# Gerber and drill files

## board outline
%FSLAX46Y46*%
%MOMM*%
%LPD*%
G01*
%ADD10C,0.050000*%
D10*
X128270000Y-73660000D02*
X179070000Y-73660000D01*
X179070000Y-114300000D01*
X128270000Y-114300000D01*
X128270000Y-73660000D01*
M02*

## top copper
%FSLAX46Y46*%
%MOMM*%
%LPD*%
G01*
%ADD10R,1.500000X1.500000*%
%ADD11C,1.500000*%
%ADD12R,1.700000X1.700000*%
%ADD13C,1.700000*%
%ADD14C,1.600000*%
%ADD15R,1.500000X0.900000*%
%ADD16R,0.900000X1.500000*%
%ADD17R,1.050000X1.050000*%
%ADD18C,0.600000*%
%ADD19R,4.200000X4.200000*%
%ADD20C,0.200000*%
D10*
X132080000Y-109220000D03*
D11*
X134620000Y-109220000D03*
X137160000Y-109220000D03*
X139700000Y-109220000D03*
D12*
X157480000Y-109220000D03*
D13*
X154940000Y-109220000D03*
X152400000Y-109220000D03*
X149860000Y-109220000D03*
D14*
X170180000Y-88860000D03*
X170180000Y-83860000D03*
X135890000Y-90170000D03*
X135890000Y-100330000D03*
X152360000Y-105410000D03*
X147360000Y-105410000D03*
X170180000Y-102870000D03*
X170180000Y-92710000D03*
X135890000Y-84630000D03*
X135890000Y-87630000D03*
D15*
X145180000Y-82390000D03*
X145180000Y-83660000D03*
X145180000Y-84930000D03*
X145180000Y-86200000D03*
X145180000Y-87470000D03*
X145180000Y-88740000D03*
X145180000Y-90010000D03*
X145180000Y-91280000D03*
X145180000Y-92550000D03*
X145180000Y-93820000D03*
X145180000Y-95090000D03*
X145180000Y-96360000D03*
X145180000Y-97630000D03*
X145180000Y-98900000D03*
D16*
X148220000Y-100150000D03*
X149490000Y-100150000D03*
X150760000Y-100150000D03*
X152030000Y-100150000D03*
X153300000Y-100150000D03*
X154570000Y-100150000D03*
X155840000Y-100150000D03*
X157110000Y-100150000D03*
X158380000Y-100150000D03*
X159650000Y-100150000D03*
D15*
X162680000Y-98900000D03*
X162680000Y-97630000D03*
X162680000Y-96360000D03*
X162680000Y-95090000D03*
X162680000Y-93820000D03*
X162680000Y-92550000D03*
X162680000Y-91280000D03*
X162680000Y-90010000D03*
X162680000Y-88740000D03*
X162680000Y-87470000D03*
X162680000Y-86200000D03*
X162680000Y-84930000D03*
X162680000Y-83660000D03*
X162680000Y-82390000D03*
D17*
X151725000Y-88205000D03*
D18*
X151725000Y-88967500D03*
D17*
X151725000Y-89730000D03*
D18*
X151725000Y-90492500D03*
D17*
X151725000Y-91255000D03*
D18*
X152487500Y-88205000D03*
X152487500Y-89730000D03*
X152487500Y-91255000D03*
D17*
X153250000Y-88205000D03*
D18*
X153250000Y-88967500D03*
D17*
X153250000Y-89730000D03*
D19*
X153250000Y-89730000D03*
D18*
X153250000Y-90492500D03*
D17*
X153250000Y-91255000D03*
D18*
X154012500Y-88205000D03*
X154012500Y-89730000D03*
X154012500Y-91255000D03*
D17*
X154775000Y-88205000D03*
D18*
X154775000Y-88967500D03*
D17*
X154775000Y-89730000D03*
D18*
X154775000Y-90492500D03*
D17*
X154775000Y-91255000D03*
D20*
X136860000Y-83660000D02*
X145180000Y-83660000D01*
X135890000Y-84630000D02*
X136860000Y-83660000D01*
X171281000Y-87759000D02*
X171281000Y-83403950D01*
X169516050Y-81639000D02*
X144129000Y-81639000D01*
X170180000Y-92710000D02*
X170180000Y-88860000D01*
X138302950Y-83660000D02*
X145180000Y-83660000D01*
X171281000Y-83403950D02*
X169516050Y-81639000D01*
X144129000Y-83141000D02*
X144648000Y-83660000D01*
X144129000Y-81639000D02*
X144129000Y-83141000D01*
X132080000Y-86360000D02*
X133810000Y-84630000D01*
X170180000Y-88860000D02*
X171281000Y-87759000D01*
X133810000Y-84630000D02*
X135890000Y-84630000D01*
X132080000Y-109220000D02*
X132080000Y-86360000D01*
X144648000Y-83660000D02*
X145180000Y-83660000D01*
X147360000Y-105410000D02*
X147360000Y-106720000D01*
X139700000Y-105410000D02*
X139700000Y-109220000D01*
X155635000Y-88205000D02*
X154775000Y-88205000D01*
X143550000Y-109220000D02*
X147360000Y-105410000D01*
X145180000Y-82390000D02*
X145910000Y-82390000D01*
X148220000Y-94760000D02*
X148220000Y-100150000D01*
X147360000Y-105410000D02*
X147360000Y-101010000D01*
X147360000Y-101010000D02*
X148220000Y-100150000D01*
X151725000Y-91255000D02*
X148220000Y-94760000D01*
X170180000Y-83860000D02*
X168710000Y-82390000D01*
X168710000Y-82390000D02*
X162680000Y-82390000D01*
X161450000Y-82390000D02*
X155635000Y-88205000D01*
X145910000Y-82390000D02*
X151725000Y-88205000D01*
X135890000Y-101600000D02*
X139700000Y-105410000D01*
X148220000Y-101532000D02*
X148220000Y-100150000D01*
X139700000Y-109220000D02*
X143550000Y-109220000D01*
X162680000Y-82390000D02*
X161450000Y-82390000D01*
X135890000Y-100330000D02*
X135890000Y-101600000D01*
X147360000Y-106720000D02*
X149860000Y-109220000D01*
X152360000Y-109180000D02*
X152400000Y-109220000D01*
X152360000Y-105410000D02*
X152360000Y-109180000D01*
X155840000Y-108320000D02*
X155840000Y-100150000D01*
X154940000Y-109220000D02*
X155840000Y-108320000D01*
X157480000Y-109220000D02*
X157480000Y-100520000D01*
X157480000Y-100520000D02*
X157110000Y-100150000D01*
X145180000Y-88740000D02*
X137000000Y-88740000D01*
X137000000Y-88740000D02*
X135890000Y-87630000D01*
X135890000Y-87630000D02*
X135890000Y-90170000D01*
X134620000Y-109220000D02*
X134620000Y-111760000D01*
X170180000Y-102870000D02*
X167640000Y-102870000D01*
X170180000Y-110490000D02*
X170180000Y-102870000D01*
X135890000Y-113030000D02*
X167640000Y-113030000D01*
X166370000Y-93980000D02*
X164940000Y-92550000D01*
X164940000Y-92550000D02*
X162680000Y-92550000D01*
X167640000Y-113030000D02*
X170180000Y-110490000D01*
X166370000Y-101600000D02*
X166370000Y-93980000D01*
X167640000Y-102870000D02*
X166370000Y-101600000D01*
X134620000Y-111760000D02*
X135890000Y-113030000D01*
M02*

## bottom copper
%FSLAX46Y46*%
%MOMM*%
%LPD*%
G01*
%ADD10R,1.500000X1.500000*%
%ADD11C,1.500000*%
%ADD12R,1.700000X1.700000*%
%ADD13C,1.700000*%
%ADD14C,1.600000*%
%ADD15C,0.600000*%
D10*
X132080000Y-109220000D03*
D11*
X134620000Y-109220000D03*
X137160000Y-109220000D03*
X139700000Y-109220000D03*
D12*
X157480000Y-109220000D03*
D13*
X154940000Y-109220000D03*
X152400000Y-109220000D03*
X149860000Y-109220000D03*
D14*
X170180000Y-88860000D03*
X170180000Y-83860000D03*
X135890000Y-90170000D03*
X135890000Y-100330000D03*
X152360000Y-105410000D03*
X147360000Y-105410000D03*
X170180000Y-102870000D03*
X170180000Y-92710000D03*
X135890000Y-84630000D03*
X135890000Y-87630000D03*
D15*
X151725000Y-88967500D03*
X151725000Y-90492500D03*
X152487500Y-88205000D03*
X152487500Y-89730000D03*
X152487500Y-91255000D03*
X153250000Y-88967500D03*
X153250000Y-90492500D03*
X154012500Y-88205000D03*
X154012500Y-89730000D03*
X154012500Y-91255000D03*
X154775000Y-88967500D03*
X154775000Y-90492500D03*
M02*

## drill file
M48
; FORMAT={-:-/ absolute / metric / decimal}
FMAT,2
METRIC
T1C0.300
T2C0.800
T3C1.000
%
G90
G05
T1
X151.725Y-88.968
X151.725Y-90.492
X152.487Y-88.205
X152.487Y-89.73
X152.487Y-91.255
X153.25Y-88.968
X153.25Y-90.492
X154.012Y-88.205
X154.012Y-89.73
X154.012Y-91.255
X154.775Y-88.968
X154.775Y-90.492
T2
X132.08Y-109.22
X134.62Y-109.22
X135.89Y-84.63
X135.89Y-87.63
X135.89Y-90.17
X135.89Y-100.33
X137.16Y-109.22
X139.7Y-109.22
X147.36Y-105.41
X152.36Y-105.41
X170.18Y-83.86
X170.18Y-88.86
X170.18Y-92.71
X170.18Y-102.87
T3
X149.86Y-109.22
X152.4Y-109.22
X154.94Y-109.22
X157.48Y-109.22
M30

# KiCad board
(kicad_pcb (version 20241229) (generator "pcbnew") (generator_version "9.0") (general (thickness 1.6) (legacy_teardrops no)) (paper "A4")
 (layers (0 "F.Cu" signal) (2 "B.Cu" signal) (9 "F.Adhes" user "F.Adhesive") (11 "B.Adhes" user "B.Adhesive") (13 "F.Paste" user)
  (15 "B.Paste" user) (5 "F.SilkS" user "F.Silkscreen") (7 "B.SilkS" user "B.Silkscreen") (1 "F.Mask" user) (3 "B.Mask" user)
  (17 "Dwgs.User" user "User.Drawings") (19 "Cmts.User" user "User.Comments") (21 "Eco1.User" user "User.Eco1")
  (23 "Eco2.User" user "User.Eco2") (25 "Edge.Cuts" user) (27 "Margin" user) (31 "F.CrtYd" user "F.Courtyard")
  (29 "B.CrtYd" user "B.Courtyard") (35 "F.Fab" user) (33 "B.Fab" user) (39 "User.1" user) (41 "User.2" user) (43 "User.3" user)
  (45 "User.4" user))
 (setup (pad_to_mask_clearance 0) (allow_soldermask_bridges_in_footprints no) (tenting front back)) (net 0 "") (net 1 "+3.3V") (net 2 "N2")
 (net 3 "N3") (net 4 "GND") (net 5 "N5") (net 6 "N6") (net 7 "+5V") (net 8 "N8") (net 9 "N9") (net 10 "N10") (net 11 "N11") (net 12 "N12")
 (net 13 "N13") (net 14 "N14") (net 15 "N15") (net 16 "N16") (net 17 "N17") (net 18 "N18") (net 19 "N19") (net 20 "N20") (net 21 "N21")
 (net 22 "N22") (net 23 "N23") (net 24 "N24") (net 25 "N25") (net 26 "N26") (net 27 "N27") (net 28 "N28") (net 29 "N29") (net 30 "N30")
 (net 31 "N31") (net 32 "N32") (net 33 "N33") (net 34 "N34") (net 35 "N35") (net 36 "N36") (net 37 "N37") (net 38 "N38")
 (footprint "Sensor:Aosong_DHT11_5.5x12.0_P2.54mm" (layer "F.Cu") (at 132.08 109.22 90)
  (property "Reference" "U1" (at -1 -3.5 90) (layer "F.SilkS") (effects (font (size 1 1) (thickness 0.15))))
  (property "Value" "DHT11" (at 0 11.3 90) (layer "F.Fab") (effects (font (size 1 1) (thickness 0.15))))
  (pad "1" thru_hole rect (at 0 0 90) (size 1.5 1.5) (drill 0.8) (layers "*.Cu" "*.Mask") (remove_unused_layers no) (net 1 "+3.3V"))
  (pad "2" thru_hole circle (at 0 2.54 90) (size 1.5 1.5) (drill 0.8) (layers "*.Cu" "*.Mask") (remove_unused_layers no) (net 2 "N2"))
  (pad "3" thru_hole circle (at 0 5.08 90) (size 1.5 1.5) (drill 0.8) (layers "*.Cu" "*.Mask") (remove_unused_layers no) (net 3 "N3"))
  (pad "4" thru_hole circle (at 0 7.62 90) (size 1.5 1.5) (drill 0.8) (layers "*.Cu" "*.Mask") (remove_unused_layers no) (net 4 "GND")))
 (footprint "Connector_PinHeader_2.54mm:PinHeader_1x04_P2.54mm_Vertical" (layer "F.Cu") (at 157.48 109.22 -90)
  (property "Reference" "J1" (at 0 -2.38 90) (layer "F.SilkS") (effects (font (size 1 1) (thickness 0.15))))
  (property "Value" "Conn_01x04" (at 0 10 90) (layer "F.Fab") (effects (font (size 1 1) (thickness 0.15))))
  (pad "1" thru_hole rect (at 0 0 270) (size 1.7 1.7) (drill 1) (layers "*.Cu" "*.Mask") (remove_unused_layers no) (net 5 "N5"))
  (pad "2" thru_hole circle (at 0 2.54 270) (size 1.7 1.7) (drill 1) (layers "*.Cu" "*.Mask") (remove_unused_layers no) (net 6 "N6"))
  (pad "3" thru_hole circle (at 0 5.08 270) (size 1.7 1.7) (drill 1) (layers "*.Cu" "*.Mask") (remove_unused_layers no) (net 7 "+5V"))
  (pad "4" thru_hole circle (at 0 7.62 270) (size 1.7 1.7) (drill 1) (layers "*.Cu" "*.Mask") (remove_unused_layers no) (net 4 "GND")))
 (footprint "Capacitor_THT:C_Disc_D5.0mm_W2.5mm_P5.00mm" (layer "F.Cu") (at 170.18 88.86 90)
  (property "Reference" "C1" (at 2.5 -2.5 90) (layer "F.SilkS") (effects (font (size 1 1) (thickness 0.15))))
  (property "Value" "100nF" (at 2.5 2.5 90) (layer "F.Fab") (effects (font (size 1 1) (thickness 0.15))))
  (pad "1" thru_hole circle (at 0 0 90) (size 1.6 1.6) (drill 0.8) (layers "*.Cu" "*.Mask") (remove_unused_layers no) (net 1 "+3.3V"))
  (pad "2" thru_hole circle (at 5 0 90) (size 1.6 1.6) (drill 0.8) (layers "*.Cu" "*.Mask") (remove_unused_layers no) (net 4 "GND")))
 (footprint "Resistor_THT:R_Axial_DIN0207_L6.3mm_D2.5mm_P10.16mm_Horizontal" (layer "F.Cu") (at 135.89 90.17 -90)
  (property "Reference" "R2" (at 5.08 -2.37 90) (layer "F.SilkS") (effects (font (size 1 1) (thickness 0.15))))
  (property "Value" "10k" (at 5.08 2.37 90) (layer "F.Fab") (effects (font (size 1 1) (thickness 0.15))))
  (pad "1" thru_hole circle (at 0 0 270) (size 1.6 1.6) (drill 0.8) (layers "*.Cu" "*.Mask") (remove_unused_layers no) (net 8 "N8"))
  (pad "2" thru_hole circle (at 10.16 0 270) (size 1.6 1.6) (drill 0.8) (layers "*.Cu" "*.Mask") (remove_unused_layers no) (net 4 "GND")))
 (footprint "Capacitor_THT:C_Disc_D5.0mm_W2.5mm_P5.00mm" (layer "F.Cu") (at 152.36 105.41 180)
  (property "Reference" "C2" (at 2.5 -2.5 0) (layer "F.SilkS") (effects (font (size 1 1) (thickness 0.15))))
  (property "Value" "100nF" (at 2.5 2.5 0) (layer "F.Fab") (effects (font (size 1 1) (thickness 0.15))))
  (pad "1" thru_hole circle (at 0 0 180) (size 1.6 1.6) (drill 0.8) (layers "*.Cu" "*.Mask") (remove_unused_layers no) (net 7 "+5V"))
  (pad "2" thru_hole circle (at 5 0 180) (size 1.6 1.6) (drill 0.8) (layers "*.Cu" "*.Mask") (remove_unused_layers no) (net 4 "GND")))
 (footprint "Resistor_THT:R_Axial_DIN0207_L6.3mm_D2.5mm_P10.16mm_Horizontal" (layer "F.Cu") (at 170.18 102.87 90)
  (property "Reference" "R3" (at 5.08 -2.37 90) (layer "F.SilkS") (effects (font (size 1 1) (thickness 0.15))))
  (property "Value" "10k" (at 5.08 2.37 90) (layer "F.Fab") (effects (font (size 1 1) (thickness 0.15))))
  (pad "1" thru_hole circle (at 0 0 90) (size 1.6 1.6) (drill 0.8) (layers "*.Cu" "*.Mask") (remove_unused_layers no) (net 2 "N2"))
  (pad "2" thru_hole circle (at 10.16 0 90) (size 1.6 1.6) (drill 0.8) (layers "*.Cu" "*.Mask") (remove_unused_layers no) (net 1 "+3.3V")))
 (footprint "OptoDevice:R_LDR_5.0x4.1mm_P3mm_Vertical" (layer "F.Cu") (at 135.89 84.63 -90)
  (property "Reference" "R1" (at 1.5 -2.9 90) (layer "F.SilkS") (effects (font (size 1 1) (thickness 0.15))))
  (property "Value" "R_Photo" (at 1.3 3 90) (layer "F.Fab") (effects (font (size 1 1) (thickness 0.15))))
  (pad "1" thru_hole circle (at 0 0 270) (size 1.6 1.6) (drill 0.8) (layers "*.Cu" "*.Mask") (remove_unused_layers no) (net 1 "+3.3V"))
  (pad "2" thru_hole circle (at 3 0 270) (size 1.6 1.6) (drill 0.8) (layers "*.Cu" "*.Mask") (remove_unused_layers no) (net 8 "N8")))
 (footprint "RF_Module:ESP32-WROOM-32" (layer "F.Cu") (at 153.93 90.64)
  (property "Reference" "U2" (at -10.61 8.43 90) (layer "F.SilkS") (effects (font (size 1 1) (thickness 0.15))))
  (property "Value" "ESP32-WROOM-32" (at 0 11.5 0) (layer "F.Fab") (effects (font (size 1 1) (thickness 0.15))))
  (pad "1" smd rect (at -8.75 -8.25) (size 1.5 0.9) (layers "F.Cu" "F.Mask" "F.Paste") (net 4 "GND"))
  (pad "2" smd rect (at -8.75 -6.98) (size 1.5 0.9) (layers "F.Cu" "F.Mask" "F.Paste") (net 1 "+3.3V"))
  (pad "3" smd rect (at -8.75 -5.71) (size 1.5 0.9) (layers "F.Cu" "F.Mask" "F.Paste") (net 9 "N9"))
  (pad "4" smd rect (at -8.75 -4.44) (size 1.5 0.9) (layers "F.Cu" "F.Mask" "F.Paste") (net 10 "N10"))
  (pad "5" smd rect (at -8.75 -3.17) (size 1.5 0.9) (layers "F.Cu" "F.Mask" "F.Paste") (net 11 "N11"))
  (pad "6" smd rect (at -8.75 -1.9) (size 1.5 0.9) (layers "F.Cu" "F.Mask" "F.Paste") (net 8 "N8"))
  (pad "7" smd rect (at -8.75 -0.63) (size 1.5 0.9) (layers "F.Cu" "F.Mask" "F.Paste") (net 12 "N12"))
  (pad "8" smd rect (at -8.75 0.64) (size 1.5 0.9) (layers "F.Cu" "F.Mask" "F.Paste") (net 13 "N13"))
  (pad "9" smd rect (at -8.75 1.91) (size 1.5 0.9) (layers "F.Cu" "F.Mask" "F.Paste") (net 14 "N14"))
  (pad "10" smd rect (at -8.75 3.18) (size 1.5 0.9) (layers "F.Cu" "F.Mask" "F.Paste") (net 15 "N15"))
  (pad "11" smd rect (at -8.75 4.45) (size 1.5 0.9) (layers "F.Cu" "F.Mask" "F.Paste") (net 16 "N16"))
  (pad "12" smd rect (at -8.75 5.72) (size 1.5 0.9) (layers "F.Cu" "F.Mask" "F.Paste") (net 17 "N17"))
  (pad "13" smd rect (at -8.75 6.99) (size 1.5 0.9) (layers "F.Cu" "F.Mask" "F.Paste") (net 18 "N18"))
  (pad "14" smd rect (at -8.75 8.26) (size 1.5 0.9) (layers "F.Cu" "F.Mask" "F.Paste") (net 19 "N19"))
  (pad "15" smd rect (at -5.71 9.51 90) (size 1.5 0.9) (layers "F.Cu" "F.Mask" "F.Paste") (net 4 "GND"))
  (pad "16" smd rect (at -4.44 9.51 90) (size 1.5 0.9) (layers "F.Cu" "F.Mask" "F.Paste") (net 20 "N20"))
  (pad "17" smd rect (at -3.17 9.51 90) (size 1.5 0.9) (layers "F.Cu" "F.Mask" "F.Paste") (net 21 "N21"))
  (pad "18" smd rect (at -1.9 9.51 90) (size 1.5 0.9) (layers "F.Cu" "F.Mask" "F.Paste") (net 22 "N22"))
  (pad "19" smd rect (at -0.63 9.51 90) (size 1.5 0.9) (layers "F.Cu" "F.Mask" "F.Paste") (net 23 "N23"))
  (pad "20" smd rect (at 0.64 9.51 90) (size 1.5 0.9) (layers "F.Cu" "F.Mask" "F.Paste") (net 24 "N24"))
  (pad "21" smd rect (at 1.91 9.51 90) (size 1.5 0.9) (layers "F.Cu" "F.Mask" "F.Paste") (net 6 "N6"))
  (pad "22" smd rect (at 3.18 9.51 90) (size 1.5 0.9) (layers "F.Cu" "F.Mask" "F.Paste") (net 5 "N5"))
  (pad "23" smd rect (at 4.45 9.51 90) (size 1.5 0.9) (layers "F.Cu" "F.Mask" "F.Paste") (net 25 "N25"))
  (pad "24" smd rect (at 5.72 9.51 90) (size 1.5 0.9) (layers "F.Cu" "F.Mask" "F.Paste") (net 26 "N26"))
  (pad "25" smd rect (at 8.75 8.26) (size 1.5 0.9) (layers "F.Cu" "F.Mask" "F.Paste") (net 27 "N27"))
  (pad "26" smd rect (at 8.75 6.99) (size 1.5 0.9) (layers "F.Cu" "F.Mask" "F.Paste") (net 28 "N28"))
  (pad "27" smd rect (at 8.75 5.72) (size 1.5 0.9) (layers "F.Cu" "F.Mask" "F.Paste") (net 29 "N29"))
  (pad "28" smd rect (at 8.75 4.45) (size 1.5 0.9) (layers "F.Cu" "F.Mask" "F.Paste") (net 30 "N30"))
  (pad "29" smd rect (at 8.75 3.18) (size 1.5 0.9) (layers "F.Cu" "F.Mask" "F.Paste") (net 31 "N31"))
  (pad "30" smd rect (at 8.75 1.91) (size 1.5 0.9) (layers "F.Cu" "F.Mask" "F.Paste") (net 2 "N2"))
  (pad "31" smd rect (at 8.75 0.64) (size 1.5 0.9) (layers "F.Cu" "F.Mask" "F.Paste") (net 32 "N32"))
  (pad "32" smd rect (at 8.75 -0.63) (size 1.5 0.9) (layers "F.Cu" "F.Mask" "F.Paste") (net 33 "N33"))
  (pad "33" smd rect (at 8.75 -1.9) (size 1.5 0.9) (layers "F.Cu" "F.Mask" "F.Paste") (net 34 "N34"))
  (pad "34" smd rect (at 8.75 -3.17) (size 1.5 0.9) (layers "F.Cu" "F.Mask" "F.Paste") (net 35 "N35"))
  (pad "35" smd rect (at 8.75 -4.44) (size 1.5 0.9) (layers "F.Cu" "F.Mask" "F.Paste") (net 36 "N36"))
  (pad "36" smd rect (at 8.75 -5.71) (size 1.5 0.9) (layers "F.Cu" "F.Mask" "F.Paste") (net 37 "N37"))
  (pad "37" smd rect (at 8.75 -6.98) (size 1.5 0.9) (layers "F.Cu" "F.Mask" "F.Paste") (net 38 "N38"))
  (pad "38" smd rect (at 8.75 -8.25) (size 1.5 0.9) (layers "F.Cu" "F.Mask" "F.Paste") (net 4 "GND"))
  (pad "39" smd rect (at -2.205 -2.435) (size 1.05 1.05) (layers "F.Cu" "F.Paste") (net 4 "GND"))
  (pad "39" thru_hole circle (at -2.205 -1.6725) (size 0.6 0.6) (drill 0.3) (layers "*.Cu" "F.Mask") (remove_unused_layers no) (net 4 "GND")
   (zone_connect 2))
  (pad "39" smd rect (at -2.205 -0.91) (size 1.05 1.05) (layers "F.Cu" "F.Paste") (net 4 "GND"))
  (pad "39" thru_hole circle (at -2.205 -0.1475) (size 0.6 0.6) (drill 0.3) (layers "*.Cu" "F.Mask") (remove_unused_layers no) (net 4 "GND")
   (zone_connect 2))
  (pad "39" smd rect (at -2.205 0.615) (size 1.05 1.05) (layers "F.Cu" "F.Paste") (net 4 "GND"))
  (pad "39" thru_hole circle (at -1.4425 -2.435) (size 0.6 0.6) (drill 0.3) (layers "*.Cu" "F.Mask") (remove_unused_layers no) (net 4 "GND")
   (zone_connect 2))
  (pad "39" thru_hole circle (at -1.4425 -0.91) (size 0.6 0.6) (drill 0.3) (layers "*.Cu" "F.Mask") (remove_unused_layers no) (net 4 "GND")
   (zone_connect 2))
  (pad "39" thru_hole circle (at -1.4425 0.615) (size 0.6 0.6) (drill 0.3) (layers "*.Cu" "F.Mask") (remove_unused_layers no) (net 4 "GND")
   (zone_connect 2))
  (pad "39" smd rect (at -0.68 -2.435) (size 1.05 1.05) (layers "F.Cu" "F.Paste") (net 4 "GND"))
  (pad "39" thru_hole circle (at -0.68 -1.6725) (size 0.6 0.6) (drill 0.3) (layers "*.Cu" "F.Mask") (remove_unused_layers no) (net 4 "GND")
   (zone_connect 2))
  (pad "39" smd rect (at -0.68 -0.91) (size 1.05 1.05) (layers "F.Cu" "F.Paste") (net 4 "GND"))
  (pad "39" smd rect (at -0.68 -0.91) (size 4.2 4.2) (layers "F.Cu" "F.Mask") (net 4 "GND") (zone_connect 2))
  (pad "39" thru_hole circle (at -0.68 -0.1475) (size 0.6 0.6) (drill 0.3) (layers "*.Cu" "F.Mask") (remove_unused_layers no) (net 4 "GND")
   (zone_connect 2))
  (pad "39" smd rect (at -0.68 0.615) (size 1.05 1.05) (layers "F.Cu" "F.Paste") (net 4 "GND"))
  (pad "39" thru_hole circle (at 0.0825 -2.435) (size 0.6 0.6) (drill 0.3) (layers "*.Cu" "F.Mask") (remove_unused_layers no) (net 4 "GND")
   (zone_connect 2))
  (pad "39" thru_hole circle (at 0.0825 -0.91) (size 0.6 0.6) (drill 0.3) (layers "*.Cu" "F.Mask") (remove_unused_layers no) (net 4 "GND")
   (zone_connect 2))
  (pad "39" thru_hole circle (at 0.0825 0.615) (size 0.6 0.6) (drill 0.3) (layers "*.Cu" "F.Mask") (remove_unused_layers no) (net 4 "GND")
   (zone_connect 2))
  (pad "39" smd rect (at 0.845 -2.435) (size 1.05 1.05) (layers "F.Cu" "F.Paste") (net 4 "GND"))
  (pad "39" thru_hole circle (at 0.845 -1.6725) (size 0.6 0.6) (drill 0.3) (layers "*.Cu" "F.Mask") (remove_unused_layers no) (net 4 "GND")
   (zone_connect 2))
  (pad "39" smd rect (at 0.845 -0.91) (size 1.05 1.05) (layers "F.Cu" "F.Paste") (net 4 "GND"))
  (pad "39" thru_hole circle (at 0.845 -0.1475) (size 0.6 0.6) (drill 0.3) (layers "*.Cu" "F.Mask") (remove_unused_layers no) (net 4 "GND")
   (zone_connect 2))
  (pad "39" smd rect (at 0.845 0.615) (size 1.05 1.05) (layers "F.Cu" "F.Paste") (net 4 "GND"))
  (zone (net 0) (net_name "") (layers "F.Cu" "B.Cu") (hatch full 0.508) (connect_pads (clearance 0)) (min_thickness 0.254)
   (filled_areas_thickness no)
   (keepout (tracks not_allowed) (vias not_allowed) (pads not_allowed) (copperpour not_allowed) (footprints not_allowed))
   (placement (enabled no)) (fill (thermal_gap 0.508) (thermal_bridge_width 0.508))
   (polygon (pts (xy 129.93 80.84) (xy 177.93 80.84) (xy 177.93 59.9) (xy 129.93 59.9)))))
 (gr_rect (start 128.27 73.66) (end 179.07 114.3) (stroke (width 0.05) (type default)) (fill no) (layer "Edge.Cuts"))
 (segment (start 136.86 83.66) (end 145.18 83.66) (width 0.2) (layer "F.Cu") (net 1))
 (segment (start 135.89 84.63) (end 136.86 83.66) (width 0.2) (layer "F.Cu") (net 1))
 (segment (start 171.281 87.759) (end 171.281 83.40395) (width 0.2) (layer "F.Cu") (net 1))
 (segment (start 169.51605 81.639) (end 144.129 81.639) (width 0.2) (layer "F.Cu") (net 1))
 (segment (start 170.18 92.71) (end 170.18 88.86) (width 0.2) (layer "F.Cu") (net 1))
 (segment (start 138.30295 83.66) (end 145.18 83.66) (width 0.2) (layer "F.Cu") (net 1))
 (segment (start 171.281 83.40395) (end 169.51605 81.639) (width 0.2) (layer "F.Cu") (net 1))
 (segment (start 144.129 83.141) (end 144.648 83.66) (width 0.2) (layer "F.Cu") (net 1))
 (segment (start 144.129 81.639) (end 144.129 83.141) (width 0.2) (layer "F.Cu") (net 1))
 (segment (start 132.08 86.36) (end 133.81 84.63) (width 0.2) (layer "F.Cu") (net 1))
 (segment (start 170.18 88.86) (end 171.281 87.759) (width 0.2) (layer "F.Cu") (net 1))
 (segment (start 133.81 84.63) (end 135.89 84.63) (width 0.2) (layer "F.Cu") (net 1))
 (segment (start 132.08 109.22) (end 132.08 86.36) (width 0.2) (layer "F.Cu") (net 1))
 (segment (start 144.648 83.66) (end 145.18 83.66) (width 0.2) (layer "F.Cu") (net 1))
 (segment (start 147.36 105.41) (end 147.36 106.72) (width 0.2) (layer "F.Cu") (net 4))
 (segment (start 139.7 105.41) (end 139.7 109.22) (width 0.2) (layer "F.Cu") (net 4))
 (segment (start 155.635 88.205) (end 154.775 88.205) (width 0.2) (layer "F.Cu") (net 4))
 (segment (start 143.55 109.22) (end 147.36 105.41) (width 0.2) (layer "F.Cu") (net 4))
 (segment (start 145.18 82.39) (end 145.91 82.39) (width 0.2) (layer "F.Cu") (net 4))
 (segment (start 148.22 94.76) (end 148.22 100.15) (width 0.2) (layer "F.Cu") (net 4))
 (segment (start 147.36 105.41) (end 147.36 101.01) (width 0.2) (layer "F.Cu") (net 4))
 (segment (start 147.36 101.01) (end 148.22 100.15) (width 0.2) (layer "F.Cu") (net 4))
 (segment (start 151.725 91.255) (end 148.22 94.76) (width 0.2) (layer "F.Cu") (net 4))
 (segment (start 170.18 83.86) (end 168.71 82.39) (width 0.2) (layer "F.Cu") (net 4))
 (segment (start 168.71 82.39) (end 162.68 82.39) (width 0.2) (layer "F.Cu") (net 4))
 (segment (start 161.45 82.39) (end 155.635 88.205) (width 0.2) (layer "F.Cu") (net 4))
 (segment (start 145.91 82.39) (end 151.725 88.205) (width 0.2) (layer "F.Cu") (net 4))
 (segment (start 135.89 101.6) (end 139.7 105.41) (width 0.2) (layer "F.Cu") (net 4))
 (segment (start 148.22 101.532) (end 148.22 100.15) (width 0.2) (layer "F.Cu") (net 4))
 (segment (start 139.7 109.22) (end 143.55 109.22) (width 0.2) (layer "F.Cu") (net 4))
 (segment (start 162.68 82.39) (end 161.45 82.39) (width 0.2) (layer "F.Cu") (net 4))
 (segment (start 135.89 100.33) (end 135.89 101.6) (width 0.2) (layer "F.Cu") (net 4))
 (segment (start 147.36 106.72) (end 149.86 109.22) (width 0.2) (layer "F.Cu") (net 4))
 (segment (start 152.36 109.18) (end 152.4 109.22) (width 0.2) (layer "F.Cu") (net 7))
 (segment (start 152.36 105.41) (end 152.36 109.18) (width 0.2) (layer "F.Cu") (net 7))
 (segment (start 155.84 108.32) (end 155.84 100.15) (width 0.2) (layer "F.Cu") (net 6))
 (segment (start 154.94 109.22) (end 155.84 108.32) (width 0.2) (layer "F.Cu") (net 6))
 (segment (start 157.48 109.22) (end 157.48 100.52) (width 0.2) (layer "F.Cu") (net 5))
 (segment (start 157.48 100.52) (end 157.11 100.15) (width 0.2) (layer "F.Cu") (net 5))
 (segment (start 145.18 88.74) (end 137 88.74) (width 0.2) (layer "F.Cu") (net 8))
 (segment (start 137 88.74) (end 135.89 87.63) (width 0.2) (layer "F.Cu") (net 8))
 (segment (start 135.89 87.63) (end 135.89 90.17) (width 0.2) (layer "F.Cu") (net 8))
 (segment (start 134.62 109.22) (end 134.62 111.76) (width 0.2) (layer "F.Cu") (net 2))
 (segment (start 170.18 102.87) (end 167.64 102.87) (width 0.2) (layer "F.Cu") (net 2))
 (segment (start 170.18 110.49) (end 170.18 102.87) (width 0.2) (layer "F.Cu") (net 2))
 (segment (start 135.89 113.03) (end 167.64 113.03) (width 0.2) (layer "F.Cu") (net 2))
 (segment (start 166.37 93.98) (end 164.94 92.55) (width 0.2) (layer "F.Cu") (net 2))
 (segment (start 164.94 92.55) (end 162.68 92.55) (width 0.2) (layer "F.Cu") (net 2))
 (segment (start 167.64 113.03) (end 170.18 110.49) (width 0.2) (layer "F.Cu") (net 2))
 (segment (start 166.37 101.6) (end 166.37 93.98) (width 0.2) (layer "F.Cu") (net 2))
 (segment (start 167.64 102.87) (end 166.37 101.6) (width 0.2) (layer "F.Cu") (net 2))
 (segment (start 134.62 111.76) (end 135.89 113.03) (width 0.2) (layer "F.Cu") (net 2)))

